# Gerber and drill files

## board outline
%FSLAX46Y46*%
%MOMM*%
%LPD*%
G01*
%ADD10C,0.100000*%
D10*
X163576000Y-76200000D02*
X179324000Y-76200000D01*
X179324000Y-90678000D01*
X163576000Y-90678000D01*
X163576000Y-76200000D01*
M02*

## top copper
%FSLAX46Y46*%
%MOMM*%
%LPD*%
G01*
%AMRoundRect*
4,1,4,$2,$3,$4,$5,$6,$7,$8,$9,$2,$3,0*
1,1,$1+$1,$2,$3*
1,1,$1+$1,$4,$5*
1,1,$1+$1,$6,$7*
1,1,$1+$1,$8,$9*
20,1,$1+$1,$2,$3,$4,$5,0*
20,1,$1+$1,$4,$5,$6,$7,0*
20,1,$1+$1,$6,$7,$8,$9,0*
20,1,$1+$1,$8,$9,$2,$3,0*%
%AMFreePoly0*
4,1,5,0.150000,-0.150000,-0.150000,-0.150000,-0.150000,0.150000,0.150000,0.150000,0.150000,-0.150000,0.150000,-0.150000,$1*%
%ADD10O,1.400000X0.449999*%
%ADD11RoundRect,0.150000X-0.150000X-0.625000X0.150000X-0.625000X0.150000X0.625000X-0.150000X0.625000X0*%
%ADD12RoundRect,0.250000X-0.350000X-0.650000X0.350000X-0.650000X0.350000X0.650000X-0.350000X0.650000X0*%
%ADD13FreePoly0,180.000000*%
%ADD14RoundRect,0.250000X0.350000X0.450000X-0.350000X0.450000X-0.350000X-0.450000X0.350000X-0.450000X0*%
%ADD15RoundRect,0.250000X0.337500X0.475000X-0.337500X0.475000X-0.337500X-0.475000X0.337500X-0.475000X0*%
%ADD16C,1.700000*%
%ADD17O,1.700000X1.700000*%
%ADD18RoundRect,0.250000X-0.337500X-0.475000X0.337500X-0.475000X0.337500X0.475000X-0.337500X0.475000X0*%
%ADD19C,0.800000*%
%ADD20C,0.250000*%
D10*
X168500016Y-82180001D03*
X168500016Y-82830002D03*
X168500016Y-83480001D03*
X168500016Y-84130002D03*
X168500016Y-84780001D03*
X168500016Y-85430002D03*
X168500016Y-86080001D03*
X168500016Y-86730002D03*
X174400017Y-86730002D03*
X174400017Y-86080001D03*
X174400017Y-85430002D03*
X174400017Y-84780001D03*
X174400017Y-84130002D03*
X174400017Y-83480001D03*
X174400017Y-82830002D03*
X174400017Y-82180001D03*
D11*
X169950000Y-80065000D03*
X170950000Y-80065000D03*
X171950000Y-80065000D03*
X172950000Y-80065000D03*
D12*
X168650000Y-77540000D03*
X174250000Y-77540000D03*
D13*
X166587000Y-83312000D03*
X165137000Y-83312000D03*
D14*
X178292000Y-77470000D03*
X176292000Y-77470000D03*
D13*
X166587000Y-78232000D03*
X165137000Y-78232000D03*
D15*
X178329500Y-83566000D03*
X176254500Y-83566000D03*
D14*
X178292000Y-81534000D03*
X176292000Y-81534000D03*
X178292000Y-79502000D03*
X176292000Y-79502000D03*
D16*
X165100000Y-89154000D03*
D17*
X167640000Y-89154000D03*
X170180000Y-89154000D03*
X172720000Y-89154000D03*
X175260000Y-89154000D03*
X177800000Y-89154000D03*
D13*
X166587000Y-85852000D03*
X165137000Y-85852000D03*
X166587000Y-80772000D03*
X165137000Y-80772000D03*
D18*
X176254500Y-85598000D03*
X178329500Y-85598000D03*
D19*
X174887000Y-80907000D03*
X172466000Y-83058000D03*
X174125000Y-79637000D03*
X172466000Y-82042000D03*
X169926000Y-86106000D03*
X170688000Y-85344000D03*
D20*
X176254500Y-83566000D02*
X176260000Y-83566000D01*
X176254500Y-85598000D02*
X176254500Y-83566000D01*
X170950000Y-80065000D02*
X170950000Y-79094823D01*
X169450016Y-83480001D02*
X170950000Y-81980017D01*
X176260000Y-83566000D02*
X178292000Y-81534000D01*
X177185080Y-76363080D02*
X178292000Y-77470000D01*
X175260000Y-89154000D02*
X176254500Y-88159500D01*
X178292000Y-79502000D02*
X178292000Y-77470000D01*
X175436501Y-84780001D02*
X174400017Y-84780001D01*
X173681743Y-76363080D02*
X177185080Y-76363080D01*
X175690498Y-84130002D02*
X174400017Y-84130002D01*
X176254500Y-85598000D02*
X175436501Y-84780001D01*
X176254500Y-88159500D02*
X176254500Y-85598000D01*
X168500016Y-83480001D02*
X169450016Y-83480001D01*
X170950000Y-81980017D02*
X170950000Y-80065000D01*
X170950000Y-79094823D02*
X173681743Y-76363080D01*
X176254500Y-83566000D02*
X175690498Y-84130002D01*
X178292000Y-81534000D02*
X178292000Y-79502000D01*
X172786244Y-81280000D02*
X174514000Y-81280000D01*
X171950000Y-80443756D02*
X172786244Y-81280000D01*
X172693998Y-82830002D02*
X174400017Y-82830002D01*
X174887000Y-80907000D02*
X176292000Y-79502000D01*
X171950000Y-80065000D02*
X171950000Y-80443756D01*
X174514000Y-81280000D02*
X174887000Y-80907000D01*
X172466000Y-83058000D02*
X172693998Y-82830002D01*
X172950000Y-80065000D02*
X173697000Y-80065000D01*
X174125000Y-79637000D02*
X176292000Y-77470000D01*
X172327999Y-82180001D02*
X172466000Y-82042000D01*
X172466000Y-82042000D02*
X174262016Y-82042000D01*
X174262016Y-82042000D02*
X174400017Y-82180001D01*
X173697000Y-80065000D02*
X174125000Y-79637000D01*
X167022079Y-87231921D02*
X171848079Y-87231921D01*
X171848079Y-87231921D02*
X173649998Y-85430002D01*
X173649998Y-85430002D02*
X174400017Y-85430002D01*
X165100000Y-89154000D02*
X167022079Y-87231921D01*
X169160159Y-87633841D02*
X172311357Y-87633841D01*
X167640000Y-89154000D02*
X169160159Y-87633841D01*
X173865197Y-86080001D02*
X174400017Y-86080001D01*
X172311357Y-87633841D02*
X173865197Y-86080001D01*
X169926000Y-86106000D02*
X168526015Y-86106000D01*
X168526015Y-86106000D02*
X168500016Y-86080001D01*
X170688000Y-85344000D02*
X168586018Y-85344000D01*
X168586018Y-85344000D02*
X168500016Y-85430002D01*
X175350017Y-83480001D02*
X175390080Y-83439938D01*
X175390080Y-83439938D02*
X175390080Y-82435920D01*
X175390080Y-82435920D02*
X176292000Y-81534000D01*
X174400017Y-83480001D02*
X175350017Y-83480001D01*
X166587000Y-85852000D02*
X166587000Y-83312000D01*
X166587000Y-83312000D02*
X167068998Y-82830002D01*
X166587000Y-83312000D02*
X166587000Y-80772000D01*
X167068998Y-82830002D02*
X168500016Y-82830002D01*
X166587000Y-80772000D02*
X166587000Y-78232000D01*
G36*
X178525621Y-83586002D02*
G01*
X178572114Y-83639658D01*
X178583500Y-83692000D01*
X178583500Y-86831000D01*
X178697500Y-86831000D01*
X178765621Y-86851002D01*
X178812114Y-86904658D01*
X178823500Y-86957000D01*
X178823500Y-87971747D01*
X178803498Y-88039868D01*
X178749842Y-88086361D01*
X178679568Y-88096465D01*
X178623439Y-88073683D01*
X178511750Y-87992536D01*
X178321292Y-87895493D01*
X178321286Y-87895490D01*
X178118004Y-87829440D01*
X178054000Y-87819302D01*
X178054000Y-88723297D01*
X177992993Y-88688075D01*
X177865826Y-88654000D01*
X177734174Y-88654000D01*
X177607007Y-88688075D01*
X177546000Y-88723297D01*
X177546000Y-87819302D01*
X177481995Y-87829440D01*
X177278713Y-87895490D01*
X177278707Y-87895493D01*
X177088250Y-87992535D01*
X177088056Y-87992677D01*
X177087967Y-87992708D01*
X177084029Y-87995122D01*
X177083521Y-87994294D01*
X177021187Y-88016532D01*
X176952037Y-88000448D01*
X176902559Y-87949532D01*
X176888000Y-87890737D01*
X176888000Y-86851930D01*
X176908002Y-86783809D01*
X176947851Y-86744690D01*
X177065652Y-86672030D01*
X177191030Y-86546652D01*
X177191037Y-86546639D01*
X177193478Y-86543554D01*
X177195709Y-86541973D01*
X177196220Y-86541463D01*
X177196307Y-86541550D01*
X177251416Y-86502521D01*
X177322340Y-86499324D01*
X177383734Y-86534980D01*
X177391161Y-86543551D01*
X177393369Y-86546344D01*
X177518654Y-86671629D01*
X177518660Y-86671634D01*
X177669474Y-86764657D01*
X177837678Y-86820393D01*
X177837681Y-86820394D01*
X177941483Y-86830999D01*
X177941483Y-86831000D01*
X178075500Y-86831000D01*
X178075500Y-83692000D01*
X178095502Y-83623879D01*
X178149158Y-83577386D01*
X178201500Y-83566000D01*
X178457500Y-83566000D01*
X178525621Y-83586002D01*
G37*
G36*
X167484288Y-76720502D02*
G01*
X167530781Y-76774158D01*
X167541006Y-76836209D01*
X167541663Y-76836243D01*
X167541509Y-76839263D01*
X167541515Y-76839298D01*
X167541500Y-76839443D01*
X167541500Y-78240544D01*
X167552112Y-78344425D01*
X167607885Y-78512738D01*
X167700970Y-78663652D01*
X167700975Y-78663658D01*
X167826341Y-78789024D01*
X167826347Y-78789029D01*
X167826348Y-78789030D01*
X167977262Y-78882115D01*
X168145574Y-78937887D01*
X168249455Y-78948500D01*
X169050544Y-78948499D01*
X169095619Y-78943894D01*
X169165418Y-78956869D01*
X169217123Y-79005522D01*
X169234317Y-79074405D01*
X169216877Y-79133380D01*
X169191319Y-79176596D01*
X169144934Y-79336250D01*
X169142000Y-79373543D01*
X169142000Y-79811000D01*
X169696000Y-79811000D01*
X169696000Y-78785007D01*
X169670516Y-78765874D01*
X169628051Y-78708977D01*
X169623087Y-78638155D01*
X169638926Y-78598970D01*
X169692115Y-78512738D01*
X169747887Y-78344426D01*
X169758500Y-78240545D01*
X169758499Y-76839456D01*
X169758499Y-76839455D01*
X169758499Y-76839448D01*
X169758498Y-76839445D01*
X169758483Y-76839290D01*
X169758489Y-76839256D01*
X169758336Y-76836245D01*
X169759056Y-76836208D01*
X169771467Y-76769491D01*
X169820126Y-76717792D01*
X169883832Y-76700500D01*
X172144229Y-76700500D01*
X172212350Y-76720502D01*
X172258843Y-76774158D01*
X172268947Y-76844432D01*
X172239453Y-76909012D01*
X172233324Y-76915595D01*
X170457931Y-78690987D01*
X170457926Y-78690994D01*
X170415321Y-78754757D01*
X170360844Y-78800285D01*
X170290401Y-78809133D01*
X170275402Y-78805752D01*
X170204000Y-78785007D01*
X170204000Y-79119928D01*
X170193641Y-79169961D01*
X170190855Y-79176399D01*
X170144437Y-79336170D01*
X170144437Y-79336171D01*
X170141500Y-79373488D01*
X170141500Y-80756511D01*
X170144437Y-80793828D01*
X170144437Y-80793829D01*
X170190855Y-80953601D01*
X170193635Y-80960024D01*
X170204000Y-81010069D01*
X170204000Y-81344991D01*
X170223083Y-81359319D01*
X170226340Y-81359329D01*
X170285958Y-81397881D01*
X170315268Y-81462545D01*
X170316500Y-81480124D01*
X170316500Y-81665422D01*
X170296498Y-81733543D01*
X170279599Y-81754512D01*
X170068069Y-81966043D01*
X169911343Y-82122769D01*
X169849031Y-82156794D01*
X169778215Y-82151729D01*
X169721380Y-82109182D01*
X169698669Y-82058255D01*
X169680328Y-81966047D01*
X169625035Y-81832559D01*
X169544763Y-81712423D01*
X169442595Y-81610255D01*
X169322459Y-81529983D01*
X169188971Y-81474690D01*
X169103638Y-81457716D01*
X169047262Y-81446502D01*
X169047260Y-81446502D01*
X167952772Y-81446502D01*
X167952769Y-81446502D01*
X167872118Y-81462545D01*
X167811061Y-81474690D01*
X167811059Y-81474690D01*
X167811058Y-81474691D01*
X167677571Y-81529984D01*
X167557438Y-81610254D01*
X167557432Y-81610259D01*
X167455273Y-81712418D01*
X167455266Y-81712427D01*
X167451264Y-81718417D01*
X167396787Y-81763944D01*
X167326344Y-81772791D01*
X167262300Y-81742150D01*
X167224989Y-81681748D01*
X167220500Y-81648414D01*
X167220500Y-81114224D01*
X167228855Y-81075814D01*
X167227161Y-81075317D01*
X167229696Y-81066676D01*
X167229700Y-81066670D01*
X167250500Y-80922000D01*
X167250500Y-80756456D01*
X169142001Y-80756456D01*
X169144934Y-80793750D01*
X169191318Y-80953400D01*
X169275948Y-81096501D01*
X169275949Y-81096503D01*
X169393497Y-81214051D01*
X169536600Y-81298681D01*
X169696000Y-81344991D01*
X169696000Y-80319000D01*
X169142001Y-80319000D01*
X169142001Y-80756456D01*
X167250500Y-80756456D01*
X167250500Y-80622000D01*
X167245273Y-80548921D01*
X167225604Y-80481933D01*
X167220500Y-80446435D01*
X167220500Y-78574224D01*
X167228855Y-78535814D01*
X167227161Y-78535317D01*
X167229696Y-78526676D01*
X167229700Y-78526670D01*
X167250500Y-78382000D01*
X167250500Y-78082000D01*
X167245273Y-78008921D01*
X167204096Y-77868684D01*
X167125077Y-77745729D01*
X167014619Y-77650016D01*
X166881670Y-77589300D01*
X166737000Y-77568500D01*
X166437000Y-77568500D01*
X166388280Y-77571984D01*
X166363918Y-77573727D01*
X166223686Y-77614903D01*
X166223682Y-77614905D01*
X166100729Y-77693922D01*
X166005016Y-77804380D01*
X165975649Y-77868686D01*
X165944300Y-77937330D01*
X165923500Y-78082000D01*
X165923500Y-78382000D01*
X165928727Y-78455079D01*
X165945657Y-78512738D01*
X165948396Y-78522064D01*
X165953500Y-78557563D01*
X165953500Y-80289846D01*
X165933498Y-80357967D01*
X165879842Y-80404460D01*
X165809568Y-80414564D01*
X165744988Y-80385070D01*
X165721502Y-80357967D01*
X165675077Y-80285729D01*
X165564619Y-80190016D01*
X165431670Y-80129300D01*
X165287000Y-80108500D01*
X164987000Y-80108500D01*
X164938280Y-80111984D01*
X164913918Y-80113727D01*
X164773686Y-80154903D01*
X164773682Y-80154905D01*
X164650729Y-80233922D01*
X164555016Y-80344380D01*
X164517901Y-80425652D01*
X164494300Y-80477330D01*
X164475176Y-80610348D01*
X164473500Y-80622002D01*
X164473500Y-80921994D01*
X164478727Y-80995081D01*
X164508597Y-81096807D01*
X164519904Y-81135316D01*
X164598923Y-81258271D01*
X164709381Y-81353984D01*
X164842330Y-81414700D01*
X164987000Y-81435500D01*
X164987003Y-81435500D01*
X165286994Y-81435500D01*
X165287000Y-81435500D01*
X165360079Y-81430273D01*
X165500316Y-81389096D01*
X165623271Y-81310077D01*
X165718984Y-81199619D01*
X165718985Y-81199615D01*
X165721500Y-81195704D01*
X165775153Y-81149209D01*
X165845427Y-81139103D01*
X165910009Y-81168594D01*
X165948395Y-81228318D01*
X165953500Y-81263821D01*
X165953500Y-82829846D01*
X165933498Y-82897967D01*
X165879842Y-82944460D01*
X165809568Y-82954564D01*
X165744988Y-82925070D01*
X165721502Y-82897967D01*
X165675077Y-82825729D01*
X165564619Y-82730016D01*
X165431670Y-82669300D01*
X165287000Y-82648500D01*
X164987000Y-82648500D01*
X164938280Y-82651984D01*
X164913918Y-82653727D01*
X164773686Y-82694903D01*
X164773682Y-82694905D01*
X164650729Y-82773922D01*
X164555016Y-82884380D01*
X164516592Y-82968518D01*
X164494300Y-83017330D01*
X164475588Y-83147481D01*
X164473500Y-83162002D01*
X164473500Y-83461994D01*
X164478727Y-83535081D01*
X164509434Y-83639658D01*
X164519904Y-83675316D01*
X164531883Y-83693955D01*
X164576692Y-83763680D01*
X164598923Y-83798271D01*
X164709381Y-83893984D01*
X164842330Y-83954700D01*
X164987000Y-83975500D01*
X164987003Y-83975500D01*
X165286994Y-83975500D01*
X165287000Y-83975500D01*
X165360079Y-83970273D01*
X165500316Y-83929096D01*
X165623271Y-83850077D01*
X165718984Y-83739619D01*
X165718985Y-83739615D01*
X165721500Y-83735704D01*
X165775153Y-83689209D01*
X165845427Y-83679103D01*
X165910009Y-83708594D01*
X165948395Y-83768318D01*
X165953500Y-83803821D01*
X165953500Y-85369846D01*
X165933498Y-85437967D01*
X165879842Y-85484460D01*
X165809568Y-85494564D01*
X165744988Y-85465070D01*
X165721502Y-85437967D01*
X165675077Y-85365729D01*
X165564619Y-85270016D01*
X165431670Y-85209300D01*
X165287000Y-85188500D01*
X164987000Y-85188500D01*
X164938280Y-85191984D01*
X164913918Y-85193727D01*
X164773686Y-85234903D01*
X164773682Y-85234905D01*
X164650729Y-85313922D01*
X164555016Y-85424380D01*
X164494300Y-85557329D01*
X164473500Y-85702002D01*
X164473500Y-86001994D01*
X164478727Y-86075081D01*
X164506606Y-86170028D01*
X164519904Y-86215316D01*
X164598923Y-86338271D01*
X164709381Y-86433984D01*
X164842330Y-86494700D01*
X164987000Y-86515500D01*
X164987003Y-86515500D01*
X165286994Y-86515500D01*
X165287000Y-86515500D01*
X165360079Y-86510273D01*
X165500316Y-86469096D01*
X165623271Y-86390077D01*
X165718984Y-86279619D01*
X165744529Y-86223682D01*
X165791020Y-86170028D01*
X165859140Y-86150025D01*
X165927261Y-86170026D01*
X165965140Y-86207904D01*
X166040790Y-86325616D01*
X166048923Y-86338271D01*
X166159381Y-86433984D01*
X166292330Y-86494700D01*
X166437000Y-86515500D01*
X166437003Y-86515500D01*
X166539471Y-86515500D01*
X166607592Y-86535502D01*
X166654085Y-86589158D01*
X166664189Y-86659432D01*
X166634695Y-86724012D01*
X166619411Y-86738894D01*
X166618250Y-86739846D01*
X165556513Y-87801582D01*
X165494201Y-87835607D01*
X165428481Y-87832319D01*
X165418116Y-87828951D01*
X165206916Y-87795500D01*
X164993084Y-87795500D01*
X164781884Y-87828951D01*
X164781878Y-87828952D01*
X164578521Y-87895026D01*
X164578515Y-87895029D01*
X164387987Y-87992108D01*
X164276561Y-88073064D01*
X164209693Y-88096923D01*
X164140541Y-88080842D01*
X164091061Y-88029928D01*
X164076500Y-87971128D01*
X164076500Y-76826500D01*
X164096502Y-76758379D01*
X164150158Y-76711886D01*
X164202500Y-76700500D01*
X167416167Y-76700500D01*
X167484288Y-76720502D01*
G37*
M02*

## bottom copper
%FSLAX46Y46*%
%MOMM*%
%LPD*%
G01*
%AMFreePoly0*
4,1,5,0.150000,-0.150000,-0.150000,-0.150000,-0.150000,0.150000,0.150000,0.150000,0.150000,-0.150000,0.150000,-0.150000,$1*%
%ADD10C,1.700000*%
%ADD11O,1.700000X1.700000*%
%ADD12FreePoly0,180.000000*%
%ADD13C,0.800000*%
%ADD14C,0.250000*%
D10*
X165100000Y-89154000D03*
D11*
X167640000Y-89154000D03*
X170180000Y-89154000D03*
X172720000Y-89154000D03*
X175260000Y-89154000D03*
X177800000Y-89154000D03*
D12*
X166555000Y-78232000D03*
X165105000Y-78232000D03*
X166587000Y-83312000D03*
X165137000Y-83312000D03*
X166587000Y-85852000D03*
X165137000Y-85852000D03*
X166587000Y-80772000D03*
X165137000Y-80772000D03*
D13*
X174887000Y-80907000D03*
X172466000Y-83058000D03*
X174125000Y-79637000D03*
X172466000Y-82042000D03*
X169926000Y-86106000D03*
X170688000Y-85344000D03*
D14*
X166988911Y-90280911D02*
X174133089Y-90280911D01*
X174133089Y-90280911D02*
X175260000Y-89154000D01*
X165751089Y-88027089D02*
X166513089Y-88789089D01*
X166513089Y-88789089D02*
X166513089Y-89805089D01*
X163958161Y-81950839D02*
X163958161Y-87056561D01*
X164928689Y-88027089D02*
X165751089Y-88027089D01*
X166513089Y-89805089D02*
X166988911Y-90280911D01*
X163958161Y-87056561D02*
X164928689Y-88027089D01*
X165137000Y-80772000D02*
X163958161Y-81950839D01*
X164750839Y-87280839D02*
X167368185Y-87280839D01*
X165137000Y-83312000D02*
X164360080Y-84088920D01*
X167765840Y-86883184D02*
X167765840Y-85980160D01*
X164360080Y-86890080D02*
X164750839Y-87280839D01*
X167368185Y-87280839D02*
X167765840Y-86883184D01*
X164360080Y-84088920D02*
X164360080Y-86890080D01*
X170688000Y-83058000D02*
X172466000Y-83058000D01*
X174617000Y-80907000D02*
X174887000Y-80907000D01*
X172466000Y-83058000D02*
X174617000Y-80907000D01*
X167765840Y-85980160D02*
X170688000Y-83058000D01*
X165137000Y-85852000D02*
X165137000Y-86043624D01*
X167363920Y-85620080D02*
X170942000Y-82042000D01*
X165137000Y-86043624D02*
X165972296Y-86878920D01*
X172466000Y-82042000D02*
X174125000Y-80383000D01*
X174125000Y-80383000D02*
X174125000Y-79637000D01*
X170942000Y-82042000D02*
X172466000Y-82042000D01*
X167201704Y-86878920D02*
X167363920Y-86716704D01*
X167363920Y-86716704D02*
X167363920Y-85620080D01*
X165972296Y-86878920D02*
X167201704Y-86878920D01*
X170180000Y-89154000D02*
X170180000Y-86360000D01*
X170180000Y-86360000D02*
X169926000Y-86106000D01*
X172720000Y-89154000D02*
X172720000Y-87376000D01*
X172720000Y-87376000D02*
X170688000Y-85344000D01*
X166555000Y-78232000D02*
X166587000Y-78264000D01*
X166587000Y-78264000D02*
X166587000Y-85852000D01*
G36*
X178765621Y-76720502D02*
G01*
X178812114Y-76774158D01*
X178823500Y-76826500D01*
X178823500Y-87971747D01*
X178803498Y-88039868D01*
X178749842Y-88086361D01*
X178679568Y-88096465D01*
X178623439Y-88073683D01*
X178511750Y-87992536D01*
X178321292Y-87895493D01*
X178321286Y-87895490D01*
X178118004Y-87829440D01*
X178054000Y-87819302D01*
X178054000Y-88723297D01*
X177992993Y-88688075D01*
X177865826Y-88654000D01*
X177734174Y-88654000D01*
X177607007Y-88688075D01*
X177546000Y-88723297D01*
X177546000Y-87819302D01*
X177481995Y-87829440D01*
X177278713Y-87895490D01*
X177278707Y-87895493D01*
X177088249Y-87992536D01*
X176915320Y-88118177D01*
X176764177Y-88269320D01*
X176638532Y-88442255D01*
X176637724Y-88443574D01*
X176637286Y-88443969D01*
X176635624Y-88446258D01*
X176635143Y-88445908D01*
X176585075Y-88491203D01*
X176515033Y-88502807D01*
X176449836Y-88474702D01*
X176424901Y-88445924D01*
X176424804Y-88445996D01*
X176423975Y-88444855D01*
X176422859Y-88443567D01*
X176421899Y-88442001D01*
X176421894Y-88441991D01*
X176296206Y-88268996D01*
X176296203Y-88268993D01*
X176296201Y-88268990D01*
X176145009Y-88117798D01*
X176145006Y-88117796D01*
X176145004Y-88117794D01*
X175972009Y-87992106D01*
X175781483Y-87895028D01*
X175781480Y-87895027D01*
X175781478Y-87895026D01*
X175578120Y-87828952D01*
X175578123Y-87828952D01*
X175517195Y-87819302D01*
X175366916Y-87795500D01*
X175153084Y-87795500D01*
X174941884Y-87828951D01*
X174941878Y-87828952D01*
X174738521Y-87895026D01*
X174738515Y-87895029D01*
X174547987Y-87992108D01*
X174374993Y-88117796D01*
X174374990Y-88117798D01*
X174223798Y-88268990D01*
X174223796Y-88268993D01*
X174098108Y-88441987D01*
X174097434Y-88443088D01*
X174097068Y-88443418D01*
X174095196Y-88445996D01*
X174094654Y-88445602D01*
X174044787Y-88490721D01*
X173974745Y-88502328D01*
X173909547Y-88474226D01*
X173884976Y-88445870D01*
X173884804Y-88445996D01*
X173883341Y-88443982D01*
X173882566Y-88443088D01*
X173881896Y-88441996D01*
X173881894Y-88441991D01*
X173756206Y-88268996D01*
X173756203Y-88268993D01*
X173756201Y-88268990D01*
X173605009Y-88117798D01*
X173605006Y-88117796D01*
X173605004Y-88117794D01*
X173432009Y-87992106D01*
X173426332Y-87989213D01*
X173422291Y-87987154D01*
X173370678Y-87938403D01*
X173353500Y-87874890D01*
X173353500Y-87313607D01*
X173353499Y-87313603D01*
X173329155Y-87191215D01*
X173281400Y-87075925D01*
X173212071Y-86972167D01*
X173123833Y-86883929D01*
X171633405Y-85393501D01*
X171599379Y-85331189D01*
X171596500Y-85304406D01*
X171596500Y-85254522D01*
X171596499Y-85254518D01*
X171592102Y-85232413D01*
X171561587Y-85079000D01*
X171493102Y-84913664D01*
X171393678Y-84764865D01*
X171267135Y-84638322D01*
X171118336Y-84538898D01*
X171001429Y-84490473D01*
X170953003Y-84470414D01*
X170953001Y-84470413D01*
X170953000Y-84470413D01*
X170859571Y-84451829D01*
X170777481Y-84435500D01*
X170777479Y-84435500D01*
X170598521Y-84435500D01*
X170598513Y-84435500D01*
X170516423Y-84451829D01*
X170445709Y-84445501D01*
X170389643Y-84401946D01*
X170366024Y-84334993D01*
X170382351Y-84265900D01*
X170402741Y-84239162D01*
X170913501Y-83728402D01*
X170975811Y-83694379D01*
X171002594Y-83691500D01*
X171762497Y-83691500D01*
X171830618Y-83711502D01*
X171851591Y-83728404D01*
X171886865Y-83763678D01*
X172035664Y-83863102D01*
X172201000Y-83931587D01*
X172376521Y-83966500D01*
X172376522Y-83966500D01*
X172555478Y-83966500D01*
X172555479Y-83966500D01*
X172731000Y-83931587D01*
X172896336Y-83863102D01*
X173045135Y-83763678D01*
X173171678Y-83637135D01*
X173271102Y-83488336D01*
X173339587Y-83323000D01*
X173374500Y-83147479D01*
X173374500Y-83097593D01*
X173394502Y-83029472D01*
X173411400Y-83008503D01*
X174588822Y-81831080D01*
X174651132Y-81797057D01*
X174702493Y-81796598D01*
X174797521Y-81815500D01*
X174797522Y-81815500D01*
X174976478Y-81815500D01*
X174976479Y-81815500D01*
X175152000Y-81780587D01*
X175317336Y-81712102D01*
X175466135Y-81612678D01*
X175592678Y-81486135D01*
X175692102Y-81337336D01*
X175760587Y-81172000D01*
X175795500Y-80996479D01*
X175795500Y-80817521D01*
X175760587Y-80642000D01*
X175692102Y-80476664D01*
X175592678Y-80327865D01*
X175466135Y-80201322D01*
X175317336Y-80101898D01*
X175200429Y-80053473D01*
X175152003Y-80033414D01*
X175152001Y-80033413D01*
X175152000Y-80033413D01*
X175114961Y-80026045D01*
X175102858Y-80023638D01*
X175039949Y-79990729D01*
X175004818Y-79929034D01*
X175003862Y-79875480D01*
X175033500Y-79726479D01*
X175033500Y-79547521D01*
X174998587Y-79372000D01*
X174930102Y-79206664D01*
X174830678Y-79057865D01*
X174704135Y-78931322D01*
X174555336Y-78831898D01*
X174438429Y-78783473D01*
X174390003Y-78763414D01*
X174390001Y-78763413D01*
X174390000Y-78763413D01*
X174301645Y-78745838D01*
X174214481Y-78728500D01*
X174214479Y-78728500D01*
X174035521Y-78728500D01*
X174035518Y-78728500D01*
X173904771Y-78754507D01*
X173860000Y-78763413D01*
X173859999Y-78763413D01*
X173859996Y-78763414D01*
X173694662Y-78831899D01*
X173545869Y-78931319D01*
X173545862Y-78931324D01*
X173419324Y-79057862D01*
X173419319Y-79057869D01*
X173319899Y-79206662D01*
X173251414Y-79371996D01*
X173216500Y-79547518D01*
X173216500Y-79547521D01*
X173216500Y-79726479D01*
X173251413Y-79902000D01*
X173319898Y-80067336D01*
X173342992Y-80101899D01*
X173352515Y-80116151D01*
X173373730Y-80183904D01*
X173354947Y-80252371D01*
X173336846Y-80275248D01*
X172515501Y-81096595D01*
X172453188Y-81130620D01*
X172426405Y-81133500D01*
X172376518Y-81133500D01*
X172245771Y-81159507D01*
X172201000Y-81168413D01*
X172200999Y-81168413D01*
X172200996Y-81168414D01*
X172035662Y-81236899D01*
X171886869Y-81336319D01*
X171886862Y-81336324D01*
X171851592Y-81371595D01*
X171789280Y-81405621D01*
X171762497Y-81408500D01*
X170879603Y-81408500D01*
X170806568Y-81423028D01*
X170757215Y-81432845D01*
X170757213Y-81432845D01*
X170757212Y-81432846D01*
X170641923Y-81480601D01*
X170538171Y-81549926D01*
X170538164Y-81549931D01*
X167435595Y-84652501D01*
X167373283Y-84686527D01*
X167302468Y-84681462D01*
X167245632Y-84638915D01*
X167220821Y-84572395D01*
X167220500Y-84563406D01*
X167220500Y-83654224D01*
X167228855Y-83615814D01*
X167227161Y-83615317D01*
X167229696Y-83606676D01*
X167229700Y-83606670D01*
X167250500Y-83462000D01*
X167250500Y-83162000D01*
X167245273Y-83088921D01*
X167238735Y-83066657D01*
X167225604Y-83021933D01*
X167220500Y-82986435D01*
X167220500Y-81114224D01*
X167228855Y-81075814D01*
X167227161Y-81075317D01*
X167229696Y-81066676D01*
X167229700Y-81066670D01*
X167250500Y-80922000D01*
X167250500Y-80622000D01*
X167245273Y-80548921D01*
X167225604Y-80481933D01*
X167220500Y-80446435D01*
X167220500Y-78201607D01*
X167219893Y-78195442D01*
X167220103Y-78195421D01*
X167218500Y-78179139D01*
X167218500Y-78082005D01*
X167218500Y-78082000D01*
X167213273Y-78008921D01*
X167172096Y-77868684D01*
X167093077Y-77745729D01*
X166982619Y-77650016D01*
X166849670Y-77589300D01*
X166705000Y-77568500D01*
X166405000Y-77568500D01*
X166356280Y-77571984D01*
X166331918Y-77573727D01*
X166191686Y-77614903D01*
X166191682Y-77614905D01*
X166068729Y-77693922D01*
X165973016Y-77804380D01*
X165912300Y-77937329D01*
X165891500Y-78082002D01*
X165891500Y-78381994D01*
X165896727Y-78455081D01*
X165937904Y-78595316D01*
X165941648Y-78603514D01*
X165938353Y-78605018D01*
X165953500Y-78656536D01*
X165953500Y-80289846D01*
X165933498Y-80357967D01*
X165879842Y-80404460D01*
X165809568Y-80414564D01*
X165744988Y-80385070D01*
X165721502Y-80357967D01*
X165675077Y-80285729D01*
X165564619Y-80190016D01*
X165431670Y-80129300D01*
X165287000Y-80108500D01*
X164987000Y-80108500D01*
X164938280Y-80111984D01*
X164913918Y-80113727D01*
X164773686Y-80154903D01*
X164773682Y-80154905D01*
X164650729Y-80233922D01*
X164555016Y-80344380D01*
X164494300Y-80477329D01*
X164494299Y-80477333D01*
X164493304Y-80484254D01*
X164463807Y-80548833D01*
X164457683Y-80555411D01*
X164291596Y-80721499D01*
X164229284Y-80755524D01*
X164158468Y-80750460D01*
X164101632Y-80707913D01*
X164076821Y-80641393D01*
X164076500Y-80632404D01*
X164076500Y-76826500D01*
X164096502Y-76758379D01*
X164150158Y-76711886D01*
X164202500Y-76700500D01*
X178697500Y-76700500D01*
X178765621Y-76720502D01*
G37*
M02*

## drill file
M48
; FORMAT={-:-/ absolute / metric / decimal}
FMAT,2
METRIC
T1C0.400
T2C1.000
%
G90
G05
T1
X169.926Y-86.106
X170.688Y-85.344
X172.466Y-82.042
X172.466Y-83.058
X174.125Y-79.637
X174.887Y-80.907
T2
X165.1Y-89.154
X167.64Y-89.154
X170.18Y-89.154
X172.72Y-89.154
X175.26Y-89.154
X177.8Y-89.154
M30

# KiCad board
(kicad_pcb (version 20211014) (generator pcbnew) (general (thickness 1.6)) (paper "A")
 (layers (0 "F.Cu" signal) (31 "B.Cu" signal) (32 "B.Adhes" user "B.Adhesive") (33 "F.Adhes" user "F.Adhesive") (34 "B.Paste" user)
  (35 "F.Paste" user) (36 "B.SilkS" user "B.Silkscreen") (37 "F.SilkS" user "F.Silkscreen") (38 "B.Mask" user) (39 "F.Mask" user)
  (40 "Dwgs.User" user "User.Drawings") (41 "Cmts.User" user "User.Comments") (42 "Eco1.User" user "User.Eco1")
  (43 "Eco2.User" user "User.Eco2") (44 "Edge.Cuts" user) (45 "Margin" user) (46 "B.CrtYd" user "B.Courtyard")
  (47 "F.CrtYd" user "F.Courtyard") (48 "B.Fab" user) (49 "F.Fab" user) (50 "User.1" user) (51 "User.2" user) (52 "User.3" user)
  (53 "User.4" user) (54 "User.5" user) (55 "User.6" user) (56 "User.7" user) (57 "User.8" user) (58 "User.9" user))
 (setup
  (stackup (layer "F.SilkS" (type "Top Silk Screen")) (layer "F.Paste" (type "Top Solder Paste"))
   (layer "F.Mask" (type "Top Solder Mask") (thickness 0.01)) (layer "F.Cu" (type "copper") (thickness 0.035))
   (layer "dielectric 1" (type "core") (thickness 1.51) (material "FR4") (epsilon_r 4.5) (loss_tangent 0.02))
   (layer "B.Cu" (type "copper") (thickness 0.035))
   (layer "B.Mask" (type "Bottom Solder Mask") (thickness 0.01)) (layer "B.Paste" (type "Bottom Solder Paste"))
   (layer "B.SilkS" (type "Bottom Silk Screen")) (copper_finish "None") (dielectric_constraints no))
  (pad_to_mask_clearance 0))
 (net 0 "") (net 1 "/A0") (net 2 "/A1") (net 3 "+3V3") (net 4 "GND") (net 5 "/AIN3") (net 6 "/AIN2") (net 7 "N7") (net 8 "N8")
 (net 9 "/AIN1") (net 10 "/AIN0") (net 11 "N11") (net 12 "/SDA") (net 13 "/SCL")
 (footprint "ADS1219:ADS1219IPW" (layer "F.Cu") (at 171.450015 84.455)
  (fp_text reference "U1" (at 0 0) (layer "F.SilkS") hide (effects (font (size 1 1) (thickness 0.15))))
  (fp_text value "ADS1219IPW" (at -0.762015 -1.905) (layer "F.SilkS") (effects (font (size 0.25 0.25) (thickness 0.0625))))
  (pad "1" smd oval (at -2.949999 -2.274999 90) (size 0.449999 1.4) (layers "F.Cu" "F.Paste" "F.Mask") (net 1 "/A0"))
  (pad "2" smd oval (at -2.949999 -1.624998 90) (size 0.449999 1.4) (layers "F.Cu" "F.Paste" "F.Mask") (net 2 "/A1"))
  (pad "3" smd oval (at -2.949999 -0.974999 90) (size 0.449999 1.4) (layers "F.Cu" "F.Paste" "F.Mask") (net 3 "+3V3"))
  (pad "4" smd oval (at -2.949999 -0.324998 90) (size 0.449999 1.4) (layers "F.Cu" "F.Paste" "F.Mask") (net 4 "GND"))
  (pad "5" smd oval (at -2.949999 0.325001 90) (size 0.449999 1.4) (layers "F.Cu" "F.Paste" "F.Mask") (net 4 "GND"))
  (pad "6" smd oval (at -2.949999 0.975002 90) (size 0.449999 1.4) (layers "F.Cu" "F.Paste" "F.Mask") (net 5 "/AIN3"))
  (pad "7" smd oval (at -2.949999 1.625001 90) (size 0.449999 1.4) (layers "F.Cu" "F.Paste" "F.Mask") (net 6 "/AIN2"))
  (pad "8" smd oval (at -2.949999 2.275002 90) (size 0.449999 1.4) (layers "F.Cu" "F.Paste" "F.Mask") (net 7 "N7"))
  (pad "9" smd oval (at 2.950002 2.275002 90) (size 0.449999 1.4) (layers "F.Cu" "F.Paste" "F.Mask") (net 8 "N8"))
  (pad "10" smd oval (at 2.950002 1.625001 90) (size 0.449999 1.4) (layers "F.Cu" "F.Paste" "F.Mask") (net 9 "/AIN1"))
  (pad "11" smd oval (at 2.950002 0.975002 90) (size 0.449999 1.4) (layers "F.Cu" "F.Paste" "F.Mask") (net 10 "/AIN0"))
  (pad "12" smd oval (at 2.950002 0.325001 90) (size 0.449999 1.4) (layers "F.Cu" "F.Paste" "F.Mask") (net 3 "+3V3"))
  (pad "13" smd oval (at 2.950002 -0.324998 90) (size 0.449999 1.4) (layers "F.Cu" "F.Paste" "F.Mask") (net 3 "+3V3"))
  (pad "14" smd oval (at 2.950002 -0.974999 90) (size 0.449999 1.4) (layers "F.Cu" "F.Paste" "F.Mask") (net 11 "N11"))
  (pad "15" smd oval (at 2.950002 -1.624998 90) (size 0.449999 1.4) (layers "F.Cu" "F.Paste" "F.Mask") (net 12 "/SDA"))
  (pad "16" smd oval (at 2.950002 -2.274999 90) (size 0.449999 1.4) (layers "F.Cu" "F.Paste" "F.Mask") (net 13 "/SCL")))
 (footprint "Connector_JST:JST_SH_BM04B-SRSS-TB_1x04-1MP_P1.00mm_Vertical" (layer "F.Cu") (at 171.45 78.74)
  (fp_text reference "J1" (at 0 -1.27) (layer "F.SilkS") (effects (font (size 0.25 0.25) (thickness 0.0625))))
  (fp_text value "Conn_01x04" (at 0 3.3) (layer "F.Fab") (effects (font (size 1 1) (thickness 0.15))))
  (pad "1" smd roundrect (at -1.5 1.325) (size 0.6 1.55) (layers "F.Cu" "F.Paste" "F.Mask") (roundrect_rratio 0.25) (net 4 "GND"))
  (pad "2" smd roundrect (at -0.5 1.325) (size 0.6 1.55) (layers "F.Cu" "F.Paste" "F.Mask") (roundrect_rratio 0.25) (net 3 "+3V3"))
  (pad "3" smd roundrect (at 0.5 1.325) (size 0.6 1.55) (layers "F.Cu" "F.Paste" "F.Mask") (roundrect_rratio 0.25) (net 12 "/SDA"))
  (pad "4" smd roundrect (at 1.5 1.325) (size 0.6 1.55) (layers "F.Cu" "F.Paste" "F.Mask") (roundrect_rratio 0.25) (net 13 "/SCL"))
  (pad "MP" smd roundrect (at -2.8 -1.2) (size 1.2 1.8) (layers "F.Cu" "F.Paste" "F.Mask") (roundrect_rratio 0.2083333333))
  (pad "MP" smd roundrect (at 2.8 -1.2) (size 1.2 1.8) (layers "F.Cu" "F.Paste" "F.Mask") (roundrect_rratio 0.2083333333)))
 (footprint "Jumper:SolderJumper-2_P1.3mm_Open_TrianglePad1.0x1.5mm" (layer "F.Cu") (at 165.862 83.312 180)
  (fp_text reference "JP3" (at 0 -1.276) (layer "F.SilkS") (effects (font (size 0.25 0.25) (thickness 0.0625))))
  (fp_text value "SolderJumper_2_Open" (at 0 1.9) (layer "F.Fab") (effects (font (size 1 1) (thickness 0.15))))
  (pad "1" smd custom (at -0.725 0 180) (size 0.3 0.3) (layers "F.Cu" "F.Mask") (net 2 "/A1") (zone_connect 2)
   (options (clearance outline) (anchor rect)) (primitives))
  (pad "2" smd custom (at 0.725 0 180) (size 0.3 0.3) (layers "F.Cu" "F.Mask") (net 12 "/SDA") (zone_connect 2)
   (options (clearance outline) (anchor rect)) (primitives)))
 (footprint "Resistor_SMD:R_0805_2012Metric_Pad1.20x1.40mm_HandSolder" (layer "F.Cu") (at 177.292 77.47 180)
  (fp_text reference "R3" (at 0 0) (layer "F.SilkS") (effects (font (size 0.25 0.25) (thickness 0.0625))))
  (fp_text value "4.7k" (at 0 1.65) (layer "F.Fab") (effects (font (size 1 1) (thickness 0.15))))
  (pad "1" smd roundrect (at -1 0 180) (size 1.2 1.4) (layers "F.Cu" "F.Paste" "F.Mask") (roundrect_rratio 0.2083333333) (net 3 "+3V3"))
  (pad "2" smd roundrect (at 1 0 180) (size 1.2 1.4) (layers "F.Cu" "F.Paste" "F.Mask") (roundrect_rratio 0.2083333333) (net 13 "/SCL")))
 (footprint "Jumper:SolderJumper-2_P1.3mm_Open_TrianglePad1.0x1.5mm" (layer "F.Cu") (at 165.862 78.232 180)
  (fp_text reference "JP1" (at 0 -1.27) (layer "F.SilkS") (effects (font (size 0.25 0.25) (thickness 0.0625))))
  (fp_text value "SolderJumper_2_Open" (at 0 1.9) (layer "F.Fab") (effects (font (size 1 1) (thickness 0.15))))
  (pad "1" smd custom (at -0.725 0 180) (size 0.3 0.3) (layers "F.Cu" "F.Mask") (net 2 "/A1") (zone_connect 2)
   (options (clearance outline) (anchor rect)) (primitives))
  (pad "2" smd custom (at 0.725 0 180) (size 0.3 0.3) (layers "F.Cu" "F.Mask") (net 4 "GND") (zone_connect 2)
   (options (clearance outline) (anchor rect)) (primitives)))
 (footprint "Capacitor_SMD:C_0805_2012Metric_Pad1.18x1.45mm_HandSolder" (layer "F.Cu") (at 177.292 83.566 180)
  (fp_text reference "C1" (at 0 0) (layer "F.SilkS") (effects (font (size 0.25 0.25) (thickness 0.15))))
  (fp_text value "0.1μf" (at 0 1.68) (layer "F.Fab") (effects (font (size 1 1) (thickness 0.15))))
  (pad "1" smd roundrect (at -1.0375 0 180) (size 1.175 1.45) (layers "F.Cu" "F.Paste" "F.Mask") (roundrect_rratio 0.2127659574)
   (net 4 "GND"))
  (pad "2" smd roundrect (at 1.0375 0 180) (size 1.175 1.45) (layers "F.Cu" "F.Paste" "F.Mask") (roundrect_rratio 0.2127659574)
   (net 3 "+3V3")))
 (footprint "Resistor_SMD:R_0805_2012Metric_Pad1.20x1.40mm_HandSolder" (layer "F.Cu") (at 177.292 81.534 180)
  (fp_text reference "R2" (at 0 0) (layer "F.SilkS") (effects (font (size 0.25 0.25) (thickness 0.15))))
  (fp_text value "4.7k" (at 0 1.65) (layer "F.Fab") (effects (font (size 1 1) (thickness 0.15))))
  (pad "1" smd roundrect (at -1 0 180) (size 1.2 1.4) (layers "F.Cu" "F.Paste" "F.Mask") (roundrect_rratio 0.2083333333) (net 3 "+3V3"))
  (pad "2" smd roundrect (at 1 0 180) (size 1.2 1.4) (layers "F.Cu" "F.Paste" "F.Mask") (roundrect_rratio 0.2083333333) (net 11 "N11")))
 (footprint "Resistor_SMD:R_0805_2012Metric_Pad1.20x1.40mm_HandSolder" (layer "F.Cu") (at 177.292 79.502 180)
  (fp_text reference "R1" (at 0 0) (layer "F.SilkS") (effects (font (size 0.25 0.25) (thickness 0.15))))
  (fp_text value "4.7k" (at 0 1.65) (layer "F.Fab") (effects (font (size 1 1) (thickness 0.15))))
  (pad "1" smd roundrect (at -1 0 180) (size 1.2 1.4) (layers "F.Cu" "F.Paste" "F.Mask") (roundrect_rratio 0.2083333333) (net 3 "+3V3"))
  (pad "2" smd roundrect (at 1 0 180) (size 1.2 1.4) (layers "F.Cu" "F.Paste" "F.Mask") (roundrect_rratio 0.2083333333) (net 12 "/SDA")))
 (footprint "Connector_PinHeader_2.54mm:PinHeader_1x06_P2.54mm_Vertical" (layer "F.Cu") (at 165.1 89.154 90)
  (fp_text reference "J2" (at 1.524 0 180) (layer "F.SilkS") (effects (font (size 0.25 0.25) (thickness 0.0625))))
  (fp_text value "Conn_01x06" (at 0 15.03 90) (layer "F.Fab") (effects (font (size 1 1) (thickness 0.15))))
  (pad "1" thru_hole circle (at 0 0 90) (size 1.7 1.7) (drill 1) (layers *.Cu *.Mask) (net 10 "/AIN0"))
  (pad "2" thru_hole oval (at 0 2.54 90) (size 1.7 1.7) (drill 1) (layers *.Cu *.Mask) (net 9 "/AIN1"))
  (pad "3" thru_hole oval (at 0 5.08 90) (size 1.7 1.7) (drill 1) (layers *.Cu *.Mask) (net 6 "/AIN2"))
  (pad "4" thru_hole oval (at 0 7.62 90) (size 1.7 1.7) (drill 1) (layers *.Cu *.Mask) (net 5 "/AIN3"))
  (pad "5" thru_hole oval (at 0 10.16 90) (size 1.7 1.7) (drill 1) (layers *.Cu *.Mask) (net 3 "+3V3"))
  (pad "6" thru_hole oval (at 0 12.7 90) (size 1.7 1.7) (drill 1) (layers *.Cu *.Mask) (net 4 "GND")))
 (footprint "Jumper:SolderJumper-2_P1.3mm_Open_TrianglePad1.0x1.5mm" (layer "F.Cu") (at 165.862 85.852 180)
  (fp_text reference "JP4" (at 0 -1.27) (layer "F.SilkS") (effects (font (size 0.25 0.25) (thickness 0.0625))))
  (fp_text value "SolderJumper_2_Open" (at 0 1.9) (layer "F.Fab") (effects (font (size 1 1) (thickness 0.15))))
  (pad "1" smd custom (at -0.725 0 180) (size 0.3 0.3) (layers "F.Cu" "F.Mask") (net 2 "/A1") (zone_connect 2)
   (options (clearance outline) (anchor rect)) (primitives))
  (pad "2" smd custom (at 0.725 0 180) (size 0.3 0.3) (layers "F.Cu" "F.Mask") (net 13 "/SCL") (zone_connect 2)
   (options (clearance outline) (anchor rect)) (primitives)))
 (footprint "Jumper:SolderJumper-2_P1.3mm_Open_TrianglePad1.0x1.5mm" (layer "F.Cu") (at 165.862 80.772 180)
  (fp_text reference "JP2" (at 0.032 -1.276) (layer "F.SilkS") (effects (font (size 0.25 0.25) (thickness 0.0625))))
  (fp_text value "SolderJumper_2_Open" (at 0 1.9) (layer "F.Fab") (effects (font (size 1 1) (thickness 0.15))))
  (pad "1" smd custom (at -0.725 0 180) (size 0.3 0.3) (layers "F.Cu" "F.Mask") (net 2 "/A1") (zone_connect 2)
   (options (clearance outline) (anchor rect)) (primitives))
  (pad "2" smd custom (at 0.725 0 180) (size 0.3 0.3) (layers "F.Cu" "F.Mask") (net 3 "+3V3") (zone_connect 2)
   (options (clearance outline) (anchor rect)) (primitives)))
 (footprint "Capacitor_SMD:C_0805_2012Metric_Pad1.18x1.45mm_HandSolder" (layer "F.Cu") (at 177.292 85.598)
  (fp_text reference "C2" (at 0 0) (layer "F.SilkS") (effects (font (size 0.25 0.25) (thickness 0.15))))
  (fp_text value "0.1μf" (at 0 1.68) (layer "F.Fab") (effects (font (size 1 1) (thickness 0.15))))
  (pad "1" smd roundrect (at -1.0375 0) (size 1.175 1.45) (layers "F.Cu" "F.Paste" "F.Mask") (roundrect_rratio 0.2127659574) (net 3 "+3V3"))
  (pad "2" smd roundrect (at 1.0375 0) (size 1.175 1.45) (layers "F.Cu" "F.Paste" "F.Mask") (roundrect_rratio 0.2127659574) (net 4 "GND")))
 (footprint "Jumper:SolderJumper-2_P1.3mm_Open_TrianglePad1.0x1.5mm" (layer "B.Cu") (at 165.83 78.232 180)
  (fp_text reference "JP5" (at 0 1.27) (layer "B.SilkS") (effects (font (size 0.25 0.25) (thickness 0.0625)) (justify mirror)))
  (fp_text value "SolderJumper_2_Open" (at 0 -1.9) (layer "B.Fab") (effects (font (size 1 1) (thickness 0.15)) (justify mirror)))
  (pad "1" smd custom (at -0.725 0 180) (size 0.3 0.3) (layers "B.Cu" "B.Mask") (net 1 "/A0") (zone_connect 2)
   (options (clearance outline) (anchor rect)) (primitives))
  (pad "2" smd custom (at 0.725 0 180) (size 0.3 0.3) (layers "B.Cu" "B.Mask") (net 4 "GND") (zone_connect 2)
   (options (clearance outline) (anchor rect)) (primitives)))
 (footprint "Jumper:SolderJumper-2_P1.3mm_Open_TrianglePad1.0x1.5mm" (layer "B.Cu") (at 165.862 83.312 180)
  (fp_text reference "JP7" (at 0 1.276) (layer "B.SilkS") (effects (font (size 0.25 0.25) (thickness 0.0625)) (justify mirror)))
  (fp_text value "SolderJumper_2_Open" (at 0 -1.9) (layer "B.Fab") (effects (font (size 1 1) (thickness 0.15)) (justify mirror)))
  (pad "1" smd custom (at -0.725 0 180) (size 0.3 0.3) (layers "B.Cu" "B.Mask") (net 1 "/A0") (zone_connect 2)
   (options (clearance outline) (anchor rect)) (primitives))
  (pad "2" smd custom (at 0.725 0 180) (size 0.3 0.3) (layers "B.Cu" "B.Mask") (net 12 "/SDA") (zone_connect 2)
   (options (clearance outline) (anchor rect)) (primitives)))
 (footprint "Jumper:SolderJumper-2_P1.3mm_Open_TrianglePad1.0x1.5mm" (layer "B.Cu") (at 165.862 85.852 180)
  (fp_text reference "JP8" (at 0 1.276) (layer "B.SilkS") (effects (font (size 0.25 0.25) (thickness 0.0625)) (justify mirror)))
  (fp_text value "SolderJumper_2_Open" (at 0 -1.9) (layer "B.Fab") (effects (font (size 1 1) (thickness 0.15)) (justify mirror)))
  (pad "1" smd custom (at -0.725 0 180) (size 0.3 0.3) (layers "B.Cu" "B.Mask") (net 1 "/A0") (zone_connect 2)
   (options (clearance outline) (anchor rect)) (primitives))
  (pad "2" smd custom (at 0.725 0 180) (size 0.3 0.3) (layers "B.Cu" "B.Mask") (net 13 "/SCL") (zone_connect 2)
   (options (clearance outline) (anchor rect)) (primitives)))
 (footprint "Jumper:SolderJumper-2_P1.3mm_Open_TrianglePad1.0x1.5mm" (layer "B.Cu") (at 165.862 80.772 180)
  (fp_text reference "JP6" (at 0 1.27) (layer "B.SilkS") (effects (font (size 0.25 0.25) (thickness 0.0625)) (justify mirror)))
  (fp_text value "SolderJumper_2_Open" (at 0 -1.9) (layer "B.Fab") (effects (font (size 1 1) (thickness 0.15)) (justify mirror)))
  (pad "1" smd custom (at -0.725 0 180) (size 0.3 0.3) (layers "B.Cu" "B.Mask") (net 1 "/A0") (zone_connect 2)
   (options (clearance outline) (anchor rect)) (primitives))
  (pad "2" smd custom (at 0.725 0 180) (size 0.3 0.3) (layers "B.Cu" "B.Mask") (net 3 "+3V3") (zone_connect 2)
   (options (clearance outline) (anchor rect)) (primitives)))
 (gr_rect (start 163.576 76.2) (end 179.324 90.678) (layer "Edge.Cuts") (width 0.1) (fill none))
 (segment (start 176.2545 83.566) (end 176.26 83.566) (width 0.25) (layer "F.Cu") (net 3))
 (segment (start 176.2545 85.598) (end 176.2545 83.566) (width 0.25) (layer "F.Cu") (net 3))
 (segment (start 170.95 80.065) (end 170.95 79.094823) (width 0.25) (layer "F.Cu") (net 3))
 (segment (start 169.450016 83.480001) (end 170.95 81.980017) (width 0.25) (layer "F.Cu") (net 3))
 (segment (start 176.26 83.566) (end 178.292 81.534) (width 0.25) (layer "F.Cu") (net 3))
 (segment (start 177.18508 76.36308) (end 178.292 77.47) (width 0.25) (layer "F.Cu") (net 3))
 (segment (start 175.26 89.154) (end 176.2545 88.1595) (width 0.25) (layer "F.Cu") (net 3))
 (segment (start 178.292 79.502) (end 178.292 77.47) (width 0.25) (layer "F.Cu") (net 3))
 (segment (start 175.436501 84.780001) (end 174.400017 84.780001) (width 0.25) (layer "F.Cu") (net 3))
 (segment (start 173.681743 76.36308) (end 177.18508 76.36308) (width 0.25) (layer "F.Cu") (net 3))
 (segment (start 175.690498 84.130002) (end 174.400017 84.130002) (width 0.25) (layer "F.Cu") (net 3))
 (segment (start 176.2545 85.598) (end 175.436501 84.780001) (width 0.25) (layer "F.Cu") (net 3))
 (segment (start 176.2545 88.1595) (end 176.2545 85.598) (width 0.25) (layer "F.Cu") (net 3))
 (segment (start 168.500016 83.480001) (end 169.450016 83.480001) (width 0.25) (layer "F.Cu") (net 3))
 (segment (start 170.95 81.980017) (end 170.95 80.065) (width 0.25) (layer "F.Cu") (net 3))
 (segment (start 170.95 79.094823) (end 173.681743 76.36308) (width 0.25) (layer "F.Cu") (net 3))
 (segment (start 176.2545 83.566) (end 175.690498 84.130002) (width 0.25) (layer "F.Cu") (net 3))
 (segment (start 178.292 81.534) (end 178.292 79.502) (width 0.25) (layer "F.Cu") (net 3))
 (segment (start 166.988911 90.280911) (end 174.133089 90.280911) (width 0.25) (layer "B.Cu") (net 3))
 (segment (start 174.133089 90.280911) (end 175.26 89.154) (width 0.25) (layer "B.Cu") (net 3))
 (segment (start 165.751089 88.027089) (end 166.513089 88.789089) (width 0.25) (layer "B.Cu") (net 3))
 (segment (start 166.513089 88.789089) (end 166.513089 89.805089) (width 0.25) (layer "B.Cu") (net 3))
 (segment (start 163.958161 81.950839) (end 163.958161 87.056561) (width 0.25) (layer "B.Cu") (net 3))
 (segment (start 164.928689 88.027089) (end 165.751089 88.027089) (width 0.25) (layer "B.Cu") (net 3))
 (segment (start 166.513089 89.805089) (end 166.988911 90.280911) (width 0.25) (layer "B.Cu") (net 3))
 (segment (start 163.958161 87.056561) (end 164.928689 88.027089) (width 0.25) (layer "B.Cu") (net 3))
 (segment (start 165.137 80.772) (end 163.958161 81.950839) (width 0.25) (layer "B.Cu") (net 3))
 (segment (start 172.786244 81.28) (end 174.514 81.28) (width 0.25) (layer "F.Cu") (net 12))
 (segment (start 171.95 80.443756) (end 172.786244 81.28) (width 0.25) (layer "F.Cu") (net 12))
 (segment (start 172.693998 82.830002) (end 174.400017 82.830002) (width 0.25) (layer "F.Cu") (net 12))
 (segment (start 174.887 80.907) (end 176.292 79.502) (width 0.25) (layer "F.Cu") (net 12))
 (segment (start 171.95 80.065) (end 171.95 80.443756) (width 0.25) (layer "F.Cu") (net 12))
 (segment (start 174.514 81.28) (end 174.887 80.907) (width 0.25) (layer "F.Cu") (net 12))
 (segment (start 172.466 83.058) (end 172.693998 82.830002) (width 0.25) (layer "F.Cu") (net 12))
 (via (at 174.887 80.907) (size 0.8) (drill 0.4) (layers "F.Cu" "B.Cu") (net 12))
 (via (at 172.466 83.058) (size 0.8) (drill 0.4) (layers "F.Cu" "B.Cu") (free) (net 12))
 (segment (start 164.750839 87.280839) (end 167.368185 87.280839) (width 0.25) (layer "B.Cu") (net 12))
 (segment (start 165.137 83.312) (end 164.36008 84.08892) (width 0.25) (layer "B.Cu") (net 12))
 (segment (start 167.76584 86.883184) (end 167.76584 85.98016) (width 0.25) (layer "B.Cu") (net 12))
 (segment (start 164.36008 86.89008) (end 164.750839 87.280839) (width 0.25) (layer "B.Cu") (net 12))
 (segment (start 167.368185 87.280839) (end 167.76584 86.883184) (width 0.25) (layer "B.Cu") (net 12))
 (segment (start 164.36008 84.08892) (end 164.36008 86.89008) (width 0.25) (layer "B.Cu") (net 12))
 (segment (start 170.688 83.058) (end 172.466 83.058) (width 0.25) (layer "B.Cu") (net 12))
 (segment (start 174.617 80.907) (end 174.887 80.907) (width 0.25) (layer "B.Cu") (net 12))
 (segment (start 172.466 83.058) (end 174.617 80.907) (width 0.25) (layer "B.Cu") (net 12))
 (segment (start 167.76584 85.98016) (end 170.688 83.058) (width 0.25) (layer "B.Cu") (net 12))
 (segment (start 172.95 80.065) (end 173.697 80.065) (width 0.25) (layer "F.Cu") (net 13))
 (segment (start 174.125 79.637) (end 176.292 77.47) (width 0.25) (layer "F.Cu") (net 13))
 (segment (start 172.327999 82.180001) (end 172.466 82.042) (width 0.25) (layer "F.Cu") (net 13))
 (segment (start 172.466 82.042) (end 174.262016 82.042) (width 0.25) (layer "F.Cu") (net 13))
 (segment (start 174.262016 82.042) (end 174.400017 82.180001) (width 0.25) (layer "F.Cu") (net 13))
 (segment (start 173.697 80.065) (end 174.125 79.637) (width 0.25) (layer "F.Cu") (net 13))
 (via (at 174.125 79.637) (size 0.8) (drill 0.4) (layers "F.Cu" "B.Cu") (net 13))
 (via (at 172.466 82.042) (size 0.8) (drill 0.4) (layers "F.Cu" "B.Cu") (free) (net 13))
 (segment (start 165.137 85.852) (end 165.137 86.043624) (width 0.25) (layer "B.Cu") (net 13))
 (segment (start 167.36392 85.62008) (end 170.942 82.042) (width 0.25) (layer "B.Cu") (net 13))
 (segment (start 165.137 86.043624) (end 165.972296 86.87892) (width 0.25) (layer "B.Cu") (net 13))
 (segment (start 172.466 82.042) (end 174.125 80.383) (width 0.25) (layer "B.Cu") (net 13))
 (segment (start 174.125 80.383) (end 174.125 79.637) (width 0.25) (layer "B.Cu") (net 13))
 (segment (start 170.942 82.042) (end 172.466 82.042) (width 0.25) (layer "B.Cu") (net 13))
 (segment (start 167.201704 86.87892) (end 167.36392 86.716704) (width 0.25) (layer "B.Cu") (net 13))
 (segment (start 167.36392 86.716704) (end 167.36392 85.62008) (width 0.25) (layer "B.Cu") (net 13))
 (segment (start 165.972296 86.87892) (end 167.201704 86.87892) (width 0.25) (layer "B.Cu") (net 13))
 (segment (start 167.022079 87.231921) (end 171.848079 87.231921) (width 0.25) (layer "F.Cu") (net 10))
 (segment (start 171.848079 87.231921) (end 173.649998 85.430002) (width 0.25) (layer "F.Cu") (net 10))
 (segment (start 173.649998 85.430002) (end 174.400017 85.430002) (width 0.25) (layer "F.Cu") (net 10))
 (segment (start 165.1 89.154) (end 167.022079 87.231921) (width 0.25) (layer "F.Cu") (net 10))
 (segment (start 169.160159 87.633841) (end 172.311357 87.633841) (width 0.25) (layer "F.Cu") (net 9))
 (segment (start 167.64 89.154) (end 169.160159 87.633841) (width 0.25) (layer "F.Cu") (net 9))
 (segment (start 173.865197 86.080001) (end 174.400017 86.080001) (width 0.25) (layer "F.Cu") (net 9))
 (segment (start 172.311357 87.633841) (end 173.865197 86.080001) (width 0.25) (layer "F.Cu") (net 9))
 (segment (start 169.926 86.106) (end 168.526015 86.106) (width 0.25) (layer "F.Cu") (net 6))
 (segment (start 168.526015 86.106) (end 168.500016 86.080001) (width 0.25) (layer "F.Cu") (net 6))
 (via (at 169.926 86.106) (size 0.8) (drill 0.4) (layers "F.Cu" "B.Cu") (free) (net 6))
 (segment (start 170.18 89.154) (end 170.18 86.36) (width 0.25) (layer "B.Cu") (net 6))
 (segment (start 170.18 86.36) (end 169.926 86.106) (width 0.25) (layer "B.Cu") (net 6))
 (segment (start 170.688 85.344) (end 168.586018 85.344) (width 0.25) (layer "F.Cu") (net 5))
 (segment (start 168.586018 85.344) (end 168.500016 85.430002) (width 0.25) (layer "F.Cu") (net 5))
 (via (at 170.688 85.344) (size 0.8) (drill 0.4) (layers "F.Cu" "B.Cu") (free) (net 5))
 (segment (start 172.72 89.154) (end 172.72 87.376) (width 0.25) (layer "B.Cu") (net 5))
 (segment (start 172.72 87.376) (end 170.688 85.344) (width 0.25) (layer "B.Cu") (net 5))
 (segment (start 175.350017 83.480001) (end 175.39008 83.439938) (width 0.25) (layer "F.Cu") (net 11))
 (segment (start 175.39008 83.439938) (end 175.39008 82.43592) (width 0.25) (layer "F.Cu") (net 11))
 (segment (start 175.39008 82.43592) (end 176.292 81.534) (width 0.25) (layer "F.Cu") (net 11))
 (segment (start 174.400017 83.480001) (end 175.350017 83.480001) (width 0.25) (layer "F.Cu") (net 11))
 (segment (start 166.587 85.852) (end 166.587 83.312) (width 0.25) (layer "F.Cu") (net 2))
 (segment (start 166.587 83.312) (end 167.068998 82.830002) (width 0.25) (layer "F.Cu") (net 2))
 (segment (start 166.587 83.312) (end 166.587 80.772) (width 0.25) (layer "F.Cu") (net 2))
 (segment (start 167.068998 82.830002) (end 168.500016 82.830002) (width 0.25) (layer "F.Cu") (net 2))
 (segment (start 166.587 80.772) (end 166.587 78.232) (width 0.25) (layer "F.Cu") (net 2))
 (segment (start 166.555 78.232) (end 166.587 78.264) (width 0.25) (layer "B.Cu") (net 1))
 (segment (start 166.587 78.264) (end 166.587 85.852) (width 0.25) (layer "B.Cu") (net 1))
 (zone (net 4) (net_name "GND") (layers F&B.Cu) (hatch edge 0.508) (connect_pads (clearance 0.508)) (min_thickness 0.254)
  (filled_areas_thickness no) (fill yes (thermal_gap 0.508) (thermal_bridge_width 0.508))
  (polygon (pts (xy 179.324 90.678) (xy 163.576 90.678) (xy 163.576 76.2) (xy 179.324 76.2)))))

